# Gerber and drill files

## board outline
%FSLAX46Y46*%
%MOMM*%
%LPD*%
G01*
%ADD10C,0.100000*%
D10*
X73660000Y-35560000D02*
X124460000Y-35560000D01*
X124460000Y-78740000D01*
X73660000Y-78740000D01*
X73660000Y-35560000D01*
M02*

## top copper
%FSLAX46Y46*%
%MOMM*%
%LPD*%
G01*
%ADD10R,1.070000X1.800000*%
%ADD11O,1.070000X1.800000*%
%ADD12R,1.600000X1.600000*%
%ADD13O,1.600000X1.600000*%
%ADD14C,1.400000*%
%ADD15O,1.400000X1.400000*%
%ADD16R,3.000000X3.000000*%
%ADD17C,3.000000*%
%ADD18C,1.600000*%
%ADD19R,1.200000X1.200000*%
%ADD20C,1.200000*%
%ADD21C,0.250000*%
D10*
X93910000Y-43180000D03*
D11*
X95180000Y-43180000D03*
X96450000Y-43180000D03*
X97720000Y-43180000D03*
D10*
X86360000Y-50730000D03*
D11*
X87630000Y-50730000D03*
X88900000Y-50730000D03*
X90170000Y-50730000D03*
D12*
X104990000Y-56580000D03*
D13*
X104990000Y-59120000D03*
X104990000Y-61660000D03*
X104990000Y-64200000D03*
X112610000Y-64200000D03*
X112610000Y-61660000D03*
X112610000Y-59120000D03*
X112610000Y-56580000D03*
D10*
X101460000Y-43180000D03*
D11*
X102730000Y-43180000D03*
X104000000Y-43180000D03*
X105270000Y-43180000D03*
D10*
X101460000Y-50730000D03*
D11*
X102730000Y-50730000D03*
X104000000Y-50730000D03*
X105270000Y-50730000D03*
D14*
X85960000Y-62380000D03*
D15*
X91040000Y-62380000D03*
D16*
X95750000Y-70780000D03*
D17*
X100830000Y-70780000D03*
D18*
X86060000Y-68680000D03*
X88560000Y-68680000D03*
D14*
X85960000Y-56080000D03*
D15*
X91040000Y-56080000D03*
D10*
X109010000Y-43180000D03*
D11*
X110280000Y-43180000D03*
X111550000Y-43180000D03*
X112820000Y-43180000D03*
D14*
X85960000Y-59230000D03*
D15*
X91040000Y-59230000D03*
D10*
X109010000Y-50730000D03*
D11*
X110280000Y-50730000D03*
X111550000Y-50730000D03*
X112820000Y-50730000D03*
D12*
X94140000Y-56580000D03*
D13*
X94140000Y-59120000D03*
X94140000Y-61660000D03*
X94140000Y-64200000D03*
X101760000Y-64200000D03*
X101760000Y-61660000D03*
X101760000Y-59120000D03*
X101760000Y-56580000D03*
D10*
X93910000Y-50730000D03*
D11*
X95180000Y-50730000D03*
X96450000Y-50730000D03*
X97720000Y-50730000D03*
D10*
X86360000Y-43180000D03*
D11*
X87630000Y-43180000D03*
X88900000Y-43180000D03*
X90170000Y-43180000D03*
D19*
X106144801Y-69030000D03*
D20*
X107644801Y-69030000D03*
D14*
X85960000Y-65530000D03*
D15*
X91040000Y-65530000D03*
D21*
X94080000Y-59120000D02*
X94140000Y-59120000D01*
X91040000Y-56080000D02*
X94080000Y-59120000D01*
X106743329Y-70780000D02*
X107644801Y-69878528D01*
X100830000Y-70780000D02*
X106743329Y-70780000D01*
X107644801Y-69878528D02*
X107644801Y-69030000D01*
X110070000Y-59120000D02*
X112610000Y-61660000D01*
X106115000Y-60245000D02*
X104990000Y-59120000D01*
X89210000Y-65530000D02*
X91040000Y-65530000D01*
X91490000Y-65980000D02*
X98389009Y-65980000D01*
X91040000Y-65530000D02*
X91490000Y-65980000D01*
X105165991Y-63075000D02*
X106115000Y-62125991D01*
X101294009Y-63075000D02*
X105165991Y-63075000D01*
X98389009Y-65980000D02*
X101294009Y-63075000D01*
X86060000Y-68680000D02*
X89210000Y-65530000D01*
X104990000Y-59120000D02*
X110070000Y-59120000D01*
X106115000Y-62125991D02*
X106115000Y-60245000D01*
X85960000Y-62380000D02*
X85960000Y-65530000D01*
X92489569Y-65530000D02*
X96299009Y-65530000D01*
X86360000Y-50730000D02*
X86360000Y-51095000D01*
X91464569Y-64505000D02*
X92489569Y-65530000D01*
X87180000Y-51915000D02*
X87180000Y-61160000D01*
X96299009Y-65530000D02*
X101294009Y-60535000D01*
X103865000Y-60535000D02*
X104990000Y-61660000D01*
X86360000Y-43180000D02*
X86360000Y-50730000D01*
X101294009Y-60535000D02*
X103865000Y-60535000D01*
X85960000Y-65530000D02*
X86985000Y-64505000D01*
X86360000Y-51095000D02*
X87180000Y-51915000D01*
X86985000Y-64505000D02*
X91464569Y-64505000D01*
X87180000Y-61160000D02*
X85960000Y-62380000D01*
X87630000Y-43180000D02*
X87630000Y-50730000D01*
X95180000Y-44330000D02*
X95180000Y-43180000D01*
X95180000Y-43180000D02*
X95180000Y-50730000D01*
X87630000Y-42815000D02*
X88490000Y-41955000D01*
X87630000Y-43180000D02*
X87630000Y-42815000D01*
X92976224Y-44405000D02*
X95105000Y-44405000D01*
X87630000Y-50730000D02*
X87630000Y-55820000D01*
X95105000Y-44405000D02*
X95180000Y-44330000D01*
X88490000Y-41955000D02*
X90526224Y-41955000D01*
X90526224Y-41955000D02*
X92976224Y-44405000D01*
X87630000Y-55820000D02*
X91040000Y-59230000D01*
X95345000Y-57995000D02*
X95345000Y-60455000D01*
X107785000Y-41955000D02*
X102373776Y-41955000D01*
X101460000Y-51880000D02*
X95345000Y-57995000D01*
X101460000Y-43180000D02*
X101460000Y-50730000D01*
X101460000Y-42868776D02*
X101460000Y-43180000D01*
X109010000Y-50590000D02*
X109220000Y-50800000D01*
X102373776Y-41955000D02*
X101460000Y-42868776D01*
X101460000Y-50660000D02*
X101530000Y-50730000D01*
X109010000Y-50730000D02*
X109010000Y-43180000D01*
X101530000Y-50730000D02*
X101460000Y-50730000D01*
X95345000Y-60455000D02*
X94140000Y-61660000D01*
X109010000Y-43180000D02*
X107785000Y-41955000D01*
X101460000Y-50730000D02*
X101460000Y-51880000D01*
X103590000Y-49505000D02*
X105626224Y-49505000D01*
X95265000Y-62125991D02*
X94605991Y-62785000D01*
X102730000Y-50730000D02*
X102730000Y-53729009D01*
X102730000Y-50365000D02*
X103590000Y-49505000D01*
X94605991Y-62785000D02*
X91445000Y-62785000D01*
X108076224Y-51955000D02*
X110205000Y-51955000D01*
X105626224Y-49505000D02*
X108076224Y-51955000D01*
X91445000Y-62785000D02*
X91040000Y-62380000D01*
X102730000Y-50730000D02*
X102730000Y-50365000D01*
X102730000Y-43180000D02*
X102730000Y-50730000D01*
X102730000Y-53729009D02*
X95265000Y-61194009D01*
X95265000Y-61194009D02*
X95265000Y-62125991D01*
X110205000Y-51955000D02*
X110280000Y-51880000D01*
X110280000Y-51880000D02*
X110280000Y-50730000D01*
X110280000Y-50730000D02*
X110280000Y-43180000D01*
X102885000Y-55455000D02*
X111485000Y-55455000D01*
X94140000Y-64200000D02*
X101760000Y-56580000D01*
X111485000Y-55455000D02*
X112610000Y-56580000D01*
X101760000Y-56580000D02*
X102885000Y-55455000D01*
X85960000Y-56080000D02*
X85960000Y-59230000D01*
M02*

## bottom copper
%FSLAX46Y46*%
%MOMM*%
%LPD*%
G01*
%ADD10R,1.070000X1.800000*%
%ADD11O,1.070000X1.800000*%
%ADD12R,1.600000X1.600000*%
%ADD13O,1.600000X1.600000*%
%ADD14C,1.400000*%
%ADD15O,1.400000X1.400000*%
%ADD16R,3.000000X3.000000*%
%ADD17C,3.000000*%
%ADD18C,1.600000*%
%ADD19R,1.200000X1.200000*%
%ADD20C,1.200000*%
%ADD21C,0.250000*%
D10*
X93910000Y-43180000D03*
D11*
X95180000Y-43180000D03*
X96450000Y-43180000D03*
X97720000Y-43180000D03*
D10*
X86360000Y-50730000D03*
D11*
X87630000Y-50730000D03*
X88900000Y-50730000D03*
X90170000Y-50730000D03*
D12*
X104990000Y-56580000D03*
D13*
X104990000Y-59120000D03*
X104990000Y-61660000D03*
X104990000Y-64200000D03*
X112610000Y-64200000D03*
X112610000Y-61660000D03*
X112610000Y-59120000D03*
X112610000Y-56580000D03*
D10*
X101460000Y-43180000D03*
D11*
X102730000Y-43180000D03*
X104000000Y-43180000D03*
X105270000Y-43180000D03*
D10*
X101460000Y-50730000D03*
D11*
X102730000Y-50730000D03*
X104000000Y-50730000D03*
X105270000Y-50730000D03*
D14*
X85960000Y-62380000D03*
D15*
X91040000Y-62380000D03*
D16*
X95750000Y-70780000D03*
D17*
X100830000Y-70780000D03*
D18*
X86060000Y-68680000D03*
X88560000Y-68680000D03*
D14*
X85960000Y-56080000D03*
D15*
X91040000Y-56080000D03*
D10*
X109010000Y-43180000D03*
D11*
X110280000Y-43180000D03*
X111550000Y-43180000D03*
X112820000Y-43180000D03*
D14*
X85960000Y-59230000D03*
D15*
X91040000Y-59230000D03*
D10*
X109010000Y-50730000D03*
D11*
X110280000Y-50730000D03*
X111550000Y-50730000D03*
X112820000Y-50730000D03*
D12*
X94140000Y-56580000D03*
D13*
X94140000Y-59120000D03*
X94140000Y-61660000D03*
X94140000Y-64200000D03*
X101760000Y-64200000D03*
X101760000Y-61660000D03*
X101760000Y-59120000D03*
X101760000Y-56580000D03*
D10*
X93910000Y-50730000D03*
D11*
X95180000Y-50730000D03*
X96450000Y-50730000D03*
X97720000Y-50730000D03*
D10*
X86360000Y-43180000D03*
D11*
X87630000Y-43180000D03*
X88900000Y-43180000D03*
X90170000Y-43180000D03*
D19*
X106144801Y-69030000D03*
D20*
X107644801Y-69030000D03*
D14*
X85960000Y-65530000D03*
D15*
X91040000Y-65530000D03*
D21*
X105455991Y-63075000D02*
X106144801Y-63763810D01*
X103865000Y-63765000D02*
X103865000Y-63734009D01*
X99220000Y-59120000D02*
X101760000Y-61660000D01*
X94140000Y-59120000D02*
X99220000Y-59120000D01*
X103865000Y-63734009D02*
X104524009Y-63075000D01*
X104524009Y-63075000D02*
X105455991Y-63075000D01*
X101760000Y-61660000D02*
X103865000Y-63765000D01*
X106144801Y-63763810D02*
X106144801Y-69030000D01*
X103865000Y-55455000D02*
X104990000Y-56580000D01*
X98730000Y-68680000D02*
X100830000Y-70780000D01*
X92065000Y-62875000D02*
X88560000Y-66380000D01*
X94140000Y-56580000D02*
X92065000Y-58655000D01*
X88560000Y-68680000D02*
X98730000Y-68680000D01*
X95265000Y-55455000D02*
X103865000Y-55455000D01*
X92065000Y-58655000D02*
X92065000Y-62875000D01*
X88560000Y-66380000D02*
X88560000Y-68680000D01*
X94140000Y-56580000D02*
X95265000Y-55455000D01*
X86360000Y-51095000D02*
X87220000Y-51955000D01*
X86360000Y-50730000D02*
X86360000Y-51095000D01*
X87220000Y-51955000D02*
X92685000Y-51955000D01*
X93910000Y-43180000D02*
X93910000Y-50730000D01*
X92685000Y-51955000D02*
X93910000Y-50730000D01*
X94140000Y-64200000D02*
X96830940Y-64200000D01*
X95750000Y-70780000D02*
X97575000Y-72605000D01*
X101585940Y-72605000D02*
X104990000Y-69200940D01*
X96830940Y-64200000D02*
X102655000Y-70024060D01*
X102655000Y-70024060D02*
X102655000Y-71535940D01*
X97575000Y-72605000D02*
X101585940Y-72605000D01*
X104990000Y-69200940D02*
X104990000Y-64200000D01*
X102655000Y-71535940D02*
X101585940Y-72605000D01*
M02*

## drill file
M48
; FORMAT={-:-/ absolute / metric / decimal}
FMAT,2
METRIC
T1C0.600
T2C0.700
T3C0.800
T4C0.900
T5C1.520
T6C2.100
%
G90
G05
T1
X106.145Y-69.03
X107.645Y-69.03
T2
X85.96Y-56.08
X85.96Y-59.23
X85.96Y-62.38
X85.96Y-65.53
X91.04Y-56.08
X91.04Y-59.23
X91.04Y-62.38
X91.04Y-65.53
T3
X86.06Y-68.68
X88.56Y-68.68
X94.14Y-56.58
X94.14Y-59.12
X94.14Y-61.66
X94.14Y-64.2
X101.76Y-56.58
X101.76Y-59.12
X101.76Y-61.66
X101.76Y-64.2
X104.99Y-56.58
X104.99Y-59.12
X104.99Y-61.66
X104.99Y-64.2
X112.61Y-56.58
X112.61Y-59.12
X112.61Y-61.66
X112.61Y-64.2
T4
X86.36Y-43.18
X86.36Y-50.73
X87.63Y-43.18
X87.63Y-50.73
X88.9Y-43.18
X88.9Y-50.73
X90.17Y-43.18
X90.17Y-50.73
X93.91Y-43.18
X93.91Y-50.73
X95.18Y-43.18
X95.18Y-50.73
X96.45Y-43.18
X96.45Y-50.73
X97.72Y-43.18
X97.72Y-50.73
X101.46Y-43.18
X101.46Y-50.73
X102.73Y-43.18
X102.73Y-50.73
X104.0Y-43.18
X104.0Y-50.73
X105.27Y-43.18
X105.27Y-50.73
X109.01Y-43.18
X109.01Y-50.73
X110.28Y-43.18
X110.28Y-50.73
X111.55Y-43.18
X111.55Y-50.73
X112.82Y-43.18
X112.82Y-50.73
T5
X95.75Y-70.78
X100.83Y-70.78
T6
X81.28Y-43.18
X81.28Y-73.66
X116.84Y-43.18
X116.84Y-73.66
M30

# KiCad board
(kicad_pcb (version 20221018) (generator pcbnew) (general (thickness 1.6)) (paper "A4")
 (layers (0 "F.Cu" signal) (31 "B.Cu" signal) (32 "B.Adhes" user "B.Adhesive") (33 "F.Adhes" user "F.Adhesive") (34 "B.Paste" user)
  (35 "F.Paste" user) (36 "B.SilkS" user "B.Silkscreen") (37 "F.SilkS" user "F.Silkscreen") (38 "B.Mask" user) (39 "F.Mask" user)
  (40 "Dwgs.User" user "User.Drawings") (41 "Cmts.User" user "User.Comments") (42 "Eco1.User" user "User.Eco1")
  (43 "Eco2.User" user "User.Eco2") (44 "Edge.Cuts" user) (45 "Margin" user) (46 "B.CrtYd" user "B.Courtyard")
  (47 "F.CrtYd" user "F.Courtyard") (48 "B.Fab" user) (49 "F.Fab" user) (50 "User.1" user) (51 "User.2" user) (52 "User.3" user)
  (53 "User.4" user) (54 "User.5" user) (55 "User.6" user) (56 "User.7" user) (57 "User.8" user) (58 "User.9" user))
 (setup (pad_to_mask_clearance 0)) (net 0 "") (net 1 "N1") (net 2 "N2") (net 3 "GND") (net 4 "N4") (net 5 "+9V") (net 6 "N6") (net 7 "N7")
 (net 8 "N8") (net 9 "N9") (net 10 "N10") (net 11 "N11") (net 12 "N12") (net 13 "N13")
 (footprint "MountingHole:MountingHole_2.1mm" (layer "F.Cu") (at 81.28 43.18)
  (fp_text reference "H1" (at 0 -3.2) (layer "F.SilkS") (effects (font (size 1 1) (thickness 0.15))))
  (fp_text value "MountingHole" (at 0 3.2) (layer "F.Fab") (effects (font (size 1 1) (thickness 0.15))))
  (pad "" np_thru_hole circle (at 0 0) (size 2.1 2.1) (drill 2.1) (layers "*.Cu" "*.Mask")))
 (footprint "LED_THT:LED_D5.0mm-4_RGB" (layer "F.Cu") (at 93.91 43.18)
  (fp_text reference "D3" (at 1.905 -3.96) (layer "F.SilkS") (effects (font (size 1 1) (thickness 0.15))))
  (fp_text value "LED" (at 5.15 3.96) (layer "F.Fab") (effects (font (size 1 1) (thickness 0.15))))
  (pad "1" thru_hole rect (at 0 0) (size 1.07 1.8) (drill 0.9) (layers "*.Cu" "*.Mask") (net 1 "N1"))
  (pad "2" thru_hole oval (at 1.27 0) (size 1.07 1.8) (drill 0.9) (layers "*.Cu" "*.Mask") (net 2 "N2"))
  (pad "3" thru_hole oval (at 2.54 0) (size 1.07 1.8) (drill 0.9) (layers "*.Cu" "*.Mask"))
  (pad "4" thru_hole oval (at 3.81 0) (size 1.07 1.8) (drill 0.9) (layers "*.Cu" "*.Mask")))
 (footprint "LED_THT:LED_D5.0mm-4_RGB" (layer "F.Cu") (at 86.36 50.73)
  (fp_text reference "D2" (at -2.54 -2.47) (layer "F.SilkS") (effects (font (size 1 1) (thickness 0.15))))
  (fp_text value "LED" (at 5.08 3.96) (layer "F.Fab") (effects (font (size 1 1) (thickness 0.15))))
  (pad "1" thru_hole rect (at 0 0) (size 1.07 1.8) (drill 0.9) (layers "*.Cu" "*.Mask") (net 1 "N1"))
  (pad "2" thru_hole oval (at 1.27 0) (size 1.07 1.8) (drill 0.9) (layers "*.Cu" "*.Mask") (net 2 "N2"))
  (pad "3" thru_hole oval (at 2.54 0) (size 1.07 1.8) (drill 0.9) (layers "*.Cu" "*.Mask"))
  (pad "4" thru_hole oval (at 3.81 0) (size 1.07 1.8) (drill 0.9) (layers "*.Cu" "*.Mask")))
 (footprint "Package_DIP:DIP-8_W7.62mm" (layer "F.Cu") (at 104.99 56.58)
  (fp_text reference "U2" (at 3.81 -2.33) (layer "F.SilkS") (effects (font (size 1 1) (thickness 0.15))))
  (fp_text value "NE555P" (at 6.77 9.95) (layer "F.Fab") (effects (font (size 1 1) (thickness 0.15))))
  (pad "1" thru_hole rect (at 0 0) (size 1.6 1.6) (drill 0.8) (layers "*.Cu" "*.Mask") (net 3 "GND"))
  (pad "2" thru_hole oval (at 0 2.54) (size 1.6 1.6) (drill 0.8) (layers "*.Cu" "*.Mask") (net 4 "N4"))
  (pad "3" thru_hole oval (at 0 5.08) (size 1.6 1.6) (drill 0.8) (layers "*.Cu" "*.Mask") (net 1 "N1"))
  (pad "4" thru_hole oval (at 0 7.62) (size 1.6 1.6) (drill 0.8) (layers "*.Cu" "*.Mask") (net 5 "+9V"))
  (pad "5" thru_hole oval (at 7.62 7.62) (size 1.6 1.6) (drill 0.8) (layers "*.Cu" "*.Mask") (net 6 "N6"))
  (pad "6" thru_hole oval (at 7.62 5.08) (size 1.6 1.6) (drill 0.8) (layers "*.Cu" "*.Mask") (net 4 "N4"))
  (pad "7" thru_hole oval (at 7.62 2.54) (size 1.6 1.6) (drill 0.8) (layers "*.Cu" "*.Mask") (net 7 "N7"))
  (pad "8" thru_hole oval (at 7.62 0) (size 1.6 1.6) (drill 0.8) (layers "*.Cu" "*.Mask") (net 5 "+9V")))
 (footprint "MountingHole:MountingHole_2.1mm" (layer "F.Cu") (at 116.84 73.66)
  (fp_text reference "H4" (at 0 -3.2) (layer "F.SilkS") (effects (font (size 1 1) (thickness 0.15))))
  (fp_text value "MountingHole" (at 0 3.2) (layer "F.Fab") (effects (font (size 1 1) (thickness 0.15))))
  (pad "" np_thru_hole circle (at 0 0) (size 2.1 2.1) (drill 2.1) (layers "*.Cu" "*.Mask")))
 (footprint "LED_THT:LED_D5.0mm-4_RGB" (layer "F.Cu") (at 101.46 43.18)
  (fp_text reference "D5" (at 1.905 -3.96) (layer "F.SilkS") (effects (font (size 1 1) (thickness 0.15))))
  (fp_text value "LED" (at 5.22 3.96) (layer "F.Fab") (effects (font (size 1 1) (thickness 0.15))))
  (pad "1" thru_hole rect (at 0 0) (size 1.07 1.8) (drill 0.9) (layers "*.Cu" "*.Mask") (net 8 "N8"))
  (pad "2" thru_hole oval (at 1.27 0) (size 1.07 1.8) (drill 0.9) (layers "*.Cu" "*.Mask") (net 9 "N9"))
  (pad "3" thru_hole oval (at 2.54 0) (size 1.07 1.8) (drill 0.9) (layers "*.Cu" "*.Mask"))
  (pad "4" thru_hole oval (at 3.81 0) (size 1.07 1.8) (drill 0.9) (layers "*.Cu" "*.Mask")))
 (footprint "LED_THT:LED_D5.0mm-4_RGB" (layer "F.Cu") (at 101.46 50.73)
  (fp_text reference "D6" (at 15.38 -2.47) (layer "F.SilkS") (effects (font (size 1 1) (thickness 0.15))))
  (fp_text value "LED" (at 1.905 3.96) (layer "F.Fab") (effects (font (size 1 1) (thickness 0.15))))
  (pad "1" thru_hole rect (at 0 0) (size 1.07 1.8) (drill 0.9) (layers "*.Cu" "*.Mask") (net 8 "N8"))
  (pad "2" thru_hole oval (at 1.27 0) (size 1.07 1.8) (drill 0.9) (layers "*.Cu" "*.Mask") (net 9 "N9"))
  (pad "3" thru_hole oval (at 2.54 0) (size 1.07 1.8) (drill 0.9) (layers "*.Cu" "*.Mask"))
  (pad "4" thru_hole oval (at 3.81 0) (size 1.07 1.8) (drill 0.9) (layers "*.Cu" "*.Mask")))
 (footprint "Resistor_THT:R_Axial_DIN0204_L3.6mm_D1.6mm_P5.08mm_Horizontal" (layer "F.Cu") (at 85.96 62.38)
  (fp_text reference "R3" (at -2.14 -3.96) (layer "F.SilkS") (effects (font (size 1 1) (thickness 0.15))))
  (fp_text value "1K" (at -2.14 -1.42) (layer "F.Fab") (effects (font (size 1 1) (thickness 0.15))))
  (pad "1" thru_hole circle (at 0 0) (size 1.4 1.4) (drill 0.7) (layers "*.Cu" "*.Mask") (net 1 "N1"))
  (pad "2" thru_hole oval (at 5.08 0) (size 1.4 1.4) (drill 0.7) (layers "*.Cu" "*.Mask") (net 9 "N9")))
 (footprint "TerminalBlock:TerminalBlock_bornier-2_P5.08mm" (layer "F.Cu") (at 95.75 70.78)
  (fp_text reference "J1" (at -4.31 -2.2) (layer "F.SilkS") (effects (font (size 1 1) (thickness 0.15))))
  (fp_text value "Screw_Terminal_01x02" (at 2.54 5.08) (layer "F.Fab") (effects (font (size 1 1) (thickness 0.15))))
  (pad "1" thru_hole rect (at 0 0) (size 3 3) (drill 1.52) (layers "*.Cu" "*.Mask") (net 5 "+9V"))
  (pad "2" thru_hole circle (at 5.08 0) (size 3 3) (drill 1.52) (layers "*.Cu" "*.Mask") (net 3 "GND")))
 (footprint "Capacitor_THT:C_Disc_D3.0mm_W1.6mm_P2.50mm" (layer "F.Cu") (at 86.06 68.68)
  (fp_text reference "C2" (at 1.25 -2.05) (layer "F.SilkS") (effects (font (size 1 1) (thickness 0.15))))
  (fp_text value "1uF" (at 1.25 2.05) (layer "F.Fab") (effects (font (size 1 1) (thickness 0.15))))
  (pad "1" thru_hole circle (at 0 0) (size 1.6 1.6) (drill 0.8) (layers "*.Cu" "*.Mask") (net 4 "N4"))
  (pad "2" thru_hole circle (at 2.5 0) (size 1.6 1.6) (drill 0.8) (layers "*.Cu" "*.Mask") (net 3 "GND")))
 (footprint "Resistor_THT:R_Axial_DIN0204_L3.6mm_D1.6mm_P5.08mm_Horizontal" (layer "F.Cu") (at 85.96 56.08)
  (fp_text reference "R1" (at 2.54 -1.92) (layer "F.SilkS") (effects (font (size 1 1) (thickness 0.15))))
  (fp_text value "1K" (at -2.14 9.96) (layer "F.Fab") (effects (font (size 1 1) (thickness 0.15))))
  (pad "1" thru_hole circle (at 0 0) (size 1.4 1.4) (drill 0.7) (layers "*.Cu" "*.Mask") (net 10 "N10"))
  (pad "2" thru_hole oval (at 5.08 0) (size 1.4 1.4) (drill 0.7) (layers "*.Cu" "*.Mask") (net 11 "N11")))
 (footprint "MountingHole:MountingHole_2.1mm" (layer "F.Cu") (at 116.84 43.18)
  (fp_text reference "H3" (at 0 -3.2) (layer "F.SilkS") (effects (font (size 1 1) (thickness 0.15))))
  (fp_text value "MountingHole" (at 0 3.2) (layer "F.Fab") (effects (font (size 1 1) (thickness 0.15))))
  (pad "" np_thru_hole circle (at 0 0) (size 2.1 2.1) (drill 2.1) (layers "*.Cu" "*.Mask")))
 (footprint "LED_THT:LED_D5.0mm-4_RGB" (layer "F.Cu") (at 109.01 43.18)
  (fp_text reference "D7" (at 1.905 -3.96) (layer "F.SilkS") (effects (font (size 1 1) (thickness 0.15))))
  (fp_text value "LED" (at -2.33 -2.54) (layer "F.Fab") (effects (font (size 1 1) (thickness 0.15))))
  (pad "1" thru_hole rect (at 0 0) (size 1.07 1.8) (drill 0.9) (layers "*.Cu" "*.Mask") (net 8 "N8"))
  (pad "2" thru_hole oval (at 1.27 0) (size 1.07 1.8) (drill 0.9) (layers "*.Cu" "*.Mask") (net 9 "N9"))
  (pad "3" thru_hole oval (at 2.54 0) (size 1.07 1.8) (drill 0.9) (layers "*.Cu" "*.Mask"))
  (pad "4" thru_hole oval (at 3.81 0) (size 1.07 1.8) (drill 0.9) (layers "*.Cu" "*.Mask")))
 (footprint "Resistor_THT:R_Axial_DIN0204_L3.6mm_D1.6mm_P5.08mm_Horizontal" (layer "F.Cu") (at 85.96 59.23)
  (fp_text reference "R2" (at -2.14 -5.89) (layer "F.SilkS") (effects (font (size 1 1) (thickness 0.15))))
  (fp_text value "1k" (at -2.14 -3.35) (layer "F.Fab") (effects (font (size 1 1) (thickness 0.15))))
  (pad "1" thru_hole circle (at 0 0) (size 1.4 1.4) (drill 0.7) (layers "*.Cu" "*.Mask") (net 10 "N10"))
  (pad "2" thru_hole oval (at 5.08 0) (size 1.4 1.4) (drill 0.7) (layers "*.Cu" "*.Mask") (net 2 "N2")))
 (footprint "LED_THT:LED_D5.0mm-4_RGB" (layer "F.Cu") (at 109.01 50.73)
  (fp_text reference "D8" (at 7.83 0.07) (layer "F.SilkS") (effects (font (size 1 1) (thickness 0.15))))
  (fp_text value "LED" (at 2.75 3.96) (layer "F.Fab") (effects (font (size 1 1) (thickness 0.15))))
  (pad "1" thru_hole rect (at 0 0) (size 1.07 1.8) (drill 0.9) (layers "*.Cu" "*.Mask") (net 8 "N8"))
  (pad "2" thru_hole oval (at 1.27 0) (size 1.07 1.8) (drill 0.9) (layers "*.Cu" "*.Mask") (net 9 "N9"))
  (pad "3" thru_hole oval (at 2.54 0) (size 1.07 1.8) (drill 0.9) (layers "*.Cu" "*.Mask"))
  (pad "4" thru_hole oval (at 3.81 0) (size 1.07 1.8) (drill 0.9) (layers "*.Cu" "*.Mask")))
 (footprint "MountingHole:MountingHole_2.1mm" (layer "F.Cu") (at 81.28 73.66)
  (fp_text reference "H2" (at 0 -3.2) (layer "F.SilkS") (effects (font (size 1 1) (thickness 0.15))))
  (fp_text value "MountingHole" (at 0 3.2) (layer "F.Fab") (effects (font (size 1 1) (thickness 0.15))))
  (pad "" np_thru_hole circle (at 0 0) (size 2.1 2.1) (drill 2.1) (layers "*.Cu" "*.Mask")))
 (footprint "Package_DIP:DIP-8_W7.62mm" (layer "F.Cu") (at 94.14 56.58)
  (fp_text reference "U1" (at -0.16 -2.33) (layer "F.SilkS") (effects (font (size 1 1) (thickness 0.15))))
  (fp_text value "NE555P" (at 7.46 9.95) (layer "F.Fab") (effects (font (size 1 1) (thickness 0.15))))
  (pad "1" thru_hole rect (at 0 0) (size 1.6 1.6) (drill 0.8) (layers "*.Cu" "*.Mask") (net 3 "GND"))
  (pad "2" thru_hole oval (at 0 2.54) (size 1.6 1.6) (drill 0.8) (layers "*.Cu" "*.Mask") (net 11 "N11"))
  (pad "3" thru_hole oval (at 0 5.08) (size 1.6 1.6) (drill 0.8) (layers "*.Cu" "*.Mask") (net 8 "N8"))
  (pad "4" thru_hole oval (at 0 7.62) (size 1.6 1.6) (drill 0.8) (layers "*.Cu" "*.Mask") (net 5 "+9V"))
  (pad "5" thru_hole oval (at 7.62 7.62) (size 1.6 1.6) (drill 0.8) (layers "*.Cu" "*.Mask") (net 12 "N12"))
  (pad "6" thru_hole oval (at 7.62 5.08) (size 1.6 1.6) (drill 0.8) (layers "*.Cu" "*.Mask") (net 11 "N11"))
  (pad "7" thru_hole oval (at 7.62 2.54) (size 1.6 1.6) (drill 0.8) (layers "*.Cu" "*.Mask") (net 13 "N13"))
  (pad "8" thru_hole oval (at 7.62 0) (size 1.6 1.6) (drill 0.8) (layers "*.Cu" "*.Mask") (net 5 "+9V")))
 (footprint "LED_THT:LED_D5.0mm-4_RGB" (layer "F.Cu") (at 93.91 50.73)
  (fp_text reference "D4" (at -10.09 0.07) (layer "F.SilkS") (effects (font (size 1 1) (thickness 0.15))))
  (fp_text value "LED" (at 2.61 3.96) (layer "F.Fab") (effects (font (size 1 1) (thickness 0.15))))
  (pad "1" thru_hole rect (at 0 0) (size 1.07 1.8) (drill 0.9) (layers "*.Cu" "*.Mask") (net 1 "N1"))
  (pad "2" thru_hole oval (at 1.27 0) (size 1.07 1.8) (drill 0.9) (layers "*.Cu" "*.Mask") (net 2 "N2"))
  (pad "3" thru_hole oval (at 2.54 0) (size 1.07 1.8) (drill 0.9) (layers "*.Cu" "*.Mask"))
  (pad "4" thru_hole oval (at 3.81 0) (size 1.07 1.8) (drill 0.9) (layers "*.Cu" "*.Mask")))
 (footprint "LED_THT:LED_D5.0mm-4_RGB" (layer "F.Cu") (at 86.36 43.18)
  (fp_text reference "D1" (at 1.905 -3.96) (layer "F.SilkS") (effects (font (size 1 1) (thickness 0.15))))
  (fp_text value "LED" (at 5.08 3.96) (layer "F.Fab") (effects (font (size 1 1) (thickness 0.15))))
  (pad "1" thru_hole rect (at 0 0) (size 1.07 1.8) (drill 0.9) (layers "*.Cu" "*.Mask") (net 1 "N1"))
  (pad "2" thru_hole oval (at 1.27 0) (size 1.07 1.8) (drill 0.9) (layers "*.Cu" "*.Mask") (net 2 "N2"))
  (pad "3" thru_hole oval (at 2.54 0) (size 1.07 1.8) (drill 0.9) (layers "*.Cu" "*.Mask"))
  (pad "4" thru_hole oval (at 3.81 0) (size 1.07 1.8) (drill 0.9) (layers "*.Cu" "*.Mask")))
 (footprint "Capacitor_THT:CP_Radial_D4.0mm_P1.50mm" (layer "F.Cu") (at 106.144801 69.03)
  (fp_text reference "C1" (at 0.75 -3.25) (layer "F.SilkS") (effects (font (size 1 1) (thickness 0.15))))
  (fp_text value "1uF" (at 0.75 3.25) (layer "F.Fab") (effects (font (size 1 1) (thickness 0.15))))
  (pad "1" thru_hole rect (at 0 0) (size 1.2 1.2) (drill 0.6) (layers "*.Cu" "*.Mask") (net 11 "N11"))
  (pad "2" thru_hole circle (at 1.5 0) (size 1.2 1.2) (drill 0.6) (layers "*.Cu" "*.Mask") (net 3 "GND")))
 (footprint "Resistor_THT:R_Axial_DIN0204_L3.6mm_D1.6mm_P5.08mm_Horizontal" (layer "F.Cu") (at 85.96 65.53)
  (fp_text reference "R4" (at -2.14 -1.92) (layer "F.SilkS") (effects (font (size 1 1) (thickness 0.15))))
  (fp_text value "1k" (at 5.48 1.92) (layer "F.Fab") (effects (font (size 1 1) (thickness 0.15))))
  (pad "1" thru_hole circle (at 0 0) (size 1.4 1.4) (drill 0.7) (layers "*.Cu" "*.Mask") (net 1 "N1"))
  (pad "2" thru_hole oval (at 5.08 0) (size 1.4 1.4) (drill 0.7) (layers "*.Cu" "*.Mask") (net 4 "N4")))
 (gr_rect (start 73.66 35.56) (end 124.46 78.74) (stroke (width 0.1) (type default)) (fill none) (layer "Edge.Cuts"))
 (segment (start 94.08 59.12) (end 94.14 59.12) (width 0.25) (layer "F.Cu") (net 11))
 (segment (start 91.04 56.08) (end 94.08 59.12) (width 0.25) (layer "F.Cu") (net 11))
 (segment (start 105.455991 63.075) (end 106.144801 63.76381) (width 0.25) (layer "B.Cu") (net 11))
 (segment (start 103.865 63.765) (end 103.865 63.734009) (width 0.25) (layer "B.Cu") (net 11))
 (segment (start 99.22 59.12) (end 101.76 61.66) (width 0.25) (layer "B.Cu") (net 11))
 (segment (start 94.14 59.12) (end 99.22 59.12) (width 0.25) (layer "B.Cu") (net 11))
 (segment (start 103.865 63.734009) (end 104.524009 63.075) (width 0.25) (layer "B.Cu") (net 11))
 (segment (start 104.524009 63.075) (end 105.455991 63.075) (width 0.25) (layer "B.Cu") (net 11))
 (segment (start 101.76 61.66) (end 103.865 63.765) (width 0.25) (layer "B.Cu") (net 11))
 (segment (start 106.144801 63.76381) (end 106.144801 69.03) (width 0.25) (layer "B.Cu") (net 11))
 (segment (start 106.743329 70.78) (end 107.644801 69.878528) (width 0.25) (layer "F.Cu") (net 3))
 (segment (start 100.83 70.78) (end 106.743329 70.78) (width 0.25) (layer "F.Cu") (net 3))
 (segment (start 107.644801 69.878528) (end 107.644801 69.03) (width 0.25) (layer "F.Cu") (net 3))
 (segment (start 103.865 55.455) (end 104.99 56.58) (width 0.25) (layer "B.Cu") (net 3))
 (segment (start 98.73 68.68) (end 100.83 70.78) (width 0.25) (layer "B.Cu") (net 3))
 (segment (start 92.065 62.875) (end 88.56 66.38) (width 0.25) (layer "B.Cu") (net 3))
 (segment (start 94.14 56.58) (end 92.065 58.655) (width 0.25) (layer "B.Cu") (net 3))
 (segment (start 88.56 68.68) (end 98.73 68.68) (width 0.25) (layer "B.Cu") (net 3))
 (segment (start 95.265 55.455) (end 103.865 55.455) (width 0.25) (layer "B.Cu") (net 3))
 (segment (start 92.065 58.655) (end 92.065 62.875) (width 0.25) (layer "B.Cu") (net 3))
 (segment (start 88.56 66.38) (end 88.56 68.68) (width 0.25) (layer "B.Cu") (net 3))
 (segment (start 94.14 56.58) (end 95.265 55.455) (width 0.25) (layer "B.Cu") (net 3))
 (segment (start 110.07 59.12) (end 112.61 61.66) (width 0.25) (layer "F.Cu") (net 4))
 (segment (start 106.115 60.245) (end 104.99 59.12) (width 0.25) (layer "F.Cu") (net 4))
 (segment (start 89.21 65.53) (end 91.04 65.53) (width 0.25) (layer "F.Cu") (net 4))
 (segment (start 91.49 65.98) (end 98.389009 65.98) (width 0.25) (layer "F.Cu") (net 4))
 (segment (start 91.04 65.53) (end 91.49 65.98) (width 0.25) (layer "F.Cu") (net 4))
 (segment (start 105.165991 63.075) (end 106.115 62.125991) (width 0.25) (layer "F.Cu") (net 4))
 (segment (start 101.294009 63.075) (end 105.165991 63.075) (width 0.25) (layer "F.Cu") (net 4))
 (segment (start 98.389009 65.98) (end 101.294009 63.075) (width 0.25) (layer "F.Cu") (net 4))
 (segment (start 86.06 68.68) (end 89.21 65.53) (width 0.25) (layer "F.Cu") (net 4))
 (segment (start 104.99 59.12) (end 110.07 59.12) (width 0.25) (layer "F.Cu") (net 4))
 (segment (start 106.115 62.125991) (end 106.115 60.245) (width 0.25) (layer "F.Cu") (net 4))
 (segment (start 85.96 62.38) (end 85.96 65.53) (width 0.25) (layer "F.Cu") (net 1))
 (segment (start 92.489569 65.53) (end 96.299009 65.53) (width 0.25) (layer "F.Cu") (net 1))
 (segment (start 86.36 50.73) (end 86.36 51.095) (width 0.25) (layer "F.Cu") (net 1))
 (segment (start 91.464569 64.505) (end 92.489569 65.53) (width 0.25) (layer "F.Cu") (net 1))
 (segment (start 87.18 51.915) (end 87.18 61.16) (width 0.25) (layer "F.Cu") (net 1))
 (segment (start 96.299009 65.53) (end 101.294009 60.535) (width 0.25) (layer "F.Cu") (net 1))
 (segment (start 103.865 60.535) (end 104.99 61.66) (width 0.25) (layer "F.Cu") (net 1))
 (segment (start 86.36 43.18) (end 86.36 50.73) (width 0.25) (layer "F.Cu") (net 1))
 (segment (start 101.294009 60.535) (end 103.865 60.535) (width 0.25) (layer "F.Cu") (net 1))
 (segment (start 85.96 65.53) (end 86.985 64.505) (width 0.25) (layer "F.Cu") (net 1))
 (segment (start 86.36 51.095) (end 87.18 51.915) (width 0.25) (layer "F.Cu") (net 1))
 (segment (start 86.985 64.505) (end 91.464569 64.505) (width 0.25) (layer "F.Cu") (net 1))
 (segment (start 87.18 61.16) (end 85.96 62.38) (width 0.25) (layer "F.Cu") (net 1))
 (segment (start 86.36 51.095) (end 87.22 51.955) (width 0.25) (layer "B.Cu") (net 1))
 (segment (start 86.36 50.73) (end 86.36 51.095) (width 0.25) (layer "B.Cu") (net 1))
 (segment (start 87.22 51.955) (end 92.685 51.955) (width 0.25) (layer "B.Cu") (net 1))
 (segment (start 93.91 43.18) (end 93.91 50.73) (width 0.25) (layer "B.Cu") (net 1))
 (segment (start 92.685 51.955) (end 93.91 50.73) (width 0.25) (layer "B.Cu") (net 1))
 (segment (start 87.63 43.18) (end 87.63 50.73) (width 0.25) (layer "F.Cu") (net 2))
 (segment (start 95.18 44.33) (end 95.18 43.18) (width 0.25) (layer "F.Cu") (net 2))
 (segment (start 95.18 43.18) (end 95.18 50.73) (width 0.25) (layer "F.Cu") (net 2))
 (segment (start 87.63 42.815) (end 88.49 41.955) (width 0.25) (layer "F.Cu") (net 2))
 (segment (start 87.63 43.18) (end 87.63 42.815) (width 0.25) (layer "F.Cu") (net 2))
 (segment (start 92.976224 44.405) (end 95.105 44.405) (width 0.25) (layer "F.Cu") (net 2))
 (segment (start 87.63 50.73) (end 87.63 55.82) (width 0.25) (layer "F.Cu") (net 2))
 (segment (start 95.105 44.405) (end 95.18 44.33) (width 0.25) (layer "F.Cu") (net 2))
 (segment (start 88.49 41.955) (end 90.526224 41.955) (width 0.25) (layer "F.Cu") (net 2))
 (segment (start 90.526224 41.955) (end 92.976224 44.405) (width 0.25) (layer "F.Cu") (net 2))
 (segment (start 87.63 55.82) (end 91.04 59.23) (width 0.25) (layer "F.Cu") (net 2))
 (segment (start 95.345 57.995) (end 95.345 60.455) (width 0.25) (layer "F.Cu") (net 8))
 (segment (start 107.785 41.955) (end 102.373776 41.955) (width 0.25) (layer "F.Cu") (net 8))
 (segment (start 101.46 51.88) (end 95.345 57.995) (width 0.25) (layer "F.Cu") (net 8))
 (segment (start 101.46 43.18) (end 101.46 50.73) (width 0.25) (layer "F.Cu") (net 8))
 (segment (start 101.46 42.868776) (end 101.46 43.18) (width 0.25) (layer "F.Cu") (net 8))
 (segment (start 109.01 50.59) (end 109.22 50.8) (width 0.25) (layer "F.Cu") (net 8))
 (segment (start 102.373776 41.955) (end 101.46 42.868776) (width 0.25) (layer "F.Cu") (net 8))
 (segment (start 101.46 50.66) (end 101.53 50.73) (width 0.25) (layer "F.Cu") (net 8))
 (segment (start 109.01 50.73) (end 109.01 43.18) (width 0.25) (layer "F.Cu") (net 8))
 (segment (start 101.53 50.73) (end 101.46 50.73) (width 0.25) (layer "F.Cu") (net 8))
 (segment (start 95.345 60.455) (end 94.14 61.66) (width 0.25) (layer "F.Cu") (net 8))
 (segment (start 109.01 43.18) (end 107.785 41.955) (width 0.25) (layer "F.Cu") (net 8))
 (segment (start 101.46 50.73) (end 101.46 51.88) (width 0.25) (layer "F.Cu") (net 8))
 (segment (start 103.59 49.505) (end 105.626224 49.505) (width 0.25) (layer "F.Cu") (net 9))
 (segment (start 95.265 62.125991) (end 94.605991 62.785) (width 0.25) (layer "F.Cu") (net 9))
 (segment (start 102.73 50.73) (end 102.73 53.729009) (width 0.25) (layer "F.Cu") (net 9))
 (segment (start 102.73 50.365) (end 103.59 49.505) (width 0.25) (layer "F.Cu") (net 9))
 (segment (start 94.605991 62.785) (end 91.445 62.785) (width 0.25) (layer "F.Cu") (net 9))
 (segment (start 108.076224 51.955) (end 110.205 51.955) (width 0.25) (layer "F.Cu") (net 9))
 (segment (start 105.626224 49.505) (end 108.076224 51.955) (width 0.25) (layer "F.Cu") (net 9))
 (segment (start 91.445 62.785) (end 91.04 62.38) (width 0.25) (layer "F.Cu") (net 9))
 (segment (start 102.73 50.73) (end 102.73 50.365) (width 0.25) (layer "F.Cu") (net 9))
 (segment (start 102.73 43.18) (end 102.73 50.73) (width 0.25) (layer "F.Cu") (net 9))
 (segment (start 102.73 53.729009) (end 95.265 61.194009) (width 0.25) (layer "F.Cu") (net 9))
 (segment (start 95.265 61.194009) (end 95.265 62.125991) (width 0.25) (layer "F.Cu") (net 9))
 (segment (start 110.205 51.955) (end 110.28 51.88) (width 0.25) (layer "F.Cu") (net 9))
 (segment (start 110.28 51.88) (end 110.28 50.73) (width 0.25) (layer "F.Cu") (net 9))
 (segment (start 110.28 50.73) (end 110.28 43.18) (width 0.25) (layer "F.Cu") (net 9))
 (segment (start 102.885 55.455) (end 111.485 55.455) (width 0.25) (layer "F.Cu") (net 5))
 (segment (start 94.14 64.2) (end 101.76 56.58) (width 0.25) (layer "F.Cu") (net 5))
 (segment (start 111.485 55.455) (end 112.61 56.58) (width 0.25) (layer "F.Cu") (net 5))
 (segment (start 101.76 56.58) (end 102.885 55.455) (width 0.25) (layer "F.Cu") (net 5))
 (segment (start 94.14 64.2) (end 96.83094 64.2) (width 0.25) (layer "B.Cu") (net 5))
 (segment (start 95.75 70.78) (end 97.575 72.605) (width 0.25) (layer "B.Cu") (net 5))
 (segment (start 101.58594 72.605) (end 104.99 69.20094) (width 0.25) (layer "B.Cu") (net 5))
 (segment (start 96.83094 64.2) (end 102.655 70.02406) (width 0.25) (layer "B.Cu") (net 5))
 (segment (start 102.655 70.02406) (end 102.655 71.53594) (width 0.25) (layer "B.Cu") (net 5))
 (segment (start 97.575 72.605) (end 101.58594 72.605) (width 0.25) (layer "B.Cu") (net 5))
 (segment (start 104.99 69.20094) (end 104.99 64.2) (width 0.25) (layer "B.Cu") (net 5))
 (segment (start 102.655 71.53594) (end 101.58594 72.605) (width 0.25) (layer "B.Cu") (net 5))
 (segment (start 85.96 56.08) (end 85.96 59.23) (width 0.25) (layer "F.Cu") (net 10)))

